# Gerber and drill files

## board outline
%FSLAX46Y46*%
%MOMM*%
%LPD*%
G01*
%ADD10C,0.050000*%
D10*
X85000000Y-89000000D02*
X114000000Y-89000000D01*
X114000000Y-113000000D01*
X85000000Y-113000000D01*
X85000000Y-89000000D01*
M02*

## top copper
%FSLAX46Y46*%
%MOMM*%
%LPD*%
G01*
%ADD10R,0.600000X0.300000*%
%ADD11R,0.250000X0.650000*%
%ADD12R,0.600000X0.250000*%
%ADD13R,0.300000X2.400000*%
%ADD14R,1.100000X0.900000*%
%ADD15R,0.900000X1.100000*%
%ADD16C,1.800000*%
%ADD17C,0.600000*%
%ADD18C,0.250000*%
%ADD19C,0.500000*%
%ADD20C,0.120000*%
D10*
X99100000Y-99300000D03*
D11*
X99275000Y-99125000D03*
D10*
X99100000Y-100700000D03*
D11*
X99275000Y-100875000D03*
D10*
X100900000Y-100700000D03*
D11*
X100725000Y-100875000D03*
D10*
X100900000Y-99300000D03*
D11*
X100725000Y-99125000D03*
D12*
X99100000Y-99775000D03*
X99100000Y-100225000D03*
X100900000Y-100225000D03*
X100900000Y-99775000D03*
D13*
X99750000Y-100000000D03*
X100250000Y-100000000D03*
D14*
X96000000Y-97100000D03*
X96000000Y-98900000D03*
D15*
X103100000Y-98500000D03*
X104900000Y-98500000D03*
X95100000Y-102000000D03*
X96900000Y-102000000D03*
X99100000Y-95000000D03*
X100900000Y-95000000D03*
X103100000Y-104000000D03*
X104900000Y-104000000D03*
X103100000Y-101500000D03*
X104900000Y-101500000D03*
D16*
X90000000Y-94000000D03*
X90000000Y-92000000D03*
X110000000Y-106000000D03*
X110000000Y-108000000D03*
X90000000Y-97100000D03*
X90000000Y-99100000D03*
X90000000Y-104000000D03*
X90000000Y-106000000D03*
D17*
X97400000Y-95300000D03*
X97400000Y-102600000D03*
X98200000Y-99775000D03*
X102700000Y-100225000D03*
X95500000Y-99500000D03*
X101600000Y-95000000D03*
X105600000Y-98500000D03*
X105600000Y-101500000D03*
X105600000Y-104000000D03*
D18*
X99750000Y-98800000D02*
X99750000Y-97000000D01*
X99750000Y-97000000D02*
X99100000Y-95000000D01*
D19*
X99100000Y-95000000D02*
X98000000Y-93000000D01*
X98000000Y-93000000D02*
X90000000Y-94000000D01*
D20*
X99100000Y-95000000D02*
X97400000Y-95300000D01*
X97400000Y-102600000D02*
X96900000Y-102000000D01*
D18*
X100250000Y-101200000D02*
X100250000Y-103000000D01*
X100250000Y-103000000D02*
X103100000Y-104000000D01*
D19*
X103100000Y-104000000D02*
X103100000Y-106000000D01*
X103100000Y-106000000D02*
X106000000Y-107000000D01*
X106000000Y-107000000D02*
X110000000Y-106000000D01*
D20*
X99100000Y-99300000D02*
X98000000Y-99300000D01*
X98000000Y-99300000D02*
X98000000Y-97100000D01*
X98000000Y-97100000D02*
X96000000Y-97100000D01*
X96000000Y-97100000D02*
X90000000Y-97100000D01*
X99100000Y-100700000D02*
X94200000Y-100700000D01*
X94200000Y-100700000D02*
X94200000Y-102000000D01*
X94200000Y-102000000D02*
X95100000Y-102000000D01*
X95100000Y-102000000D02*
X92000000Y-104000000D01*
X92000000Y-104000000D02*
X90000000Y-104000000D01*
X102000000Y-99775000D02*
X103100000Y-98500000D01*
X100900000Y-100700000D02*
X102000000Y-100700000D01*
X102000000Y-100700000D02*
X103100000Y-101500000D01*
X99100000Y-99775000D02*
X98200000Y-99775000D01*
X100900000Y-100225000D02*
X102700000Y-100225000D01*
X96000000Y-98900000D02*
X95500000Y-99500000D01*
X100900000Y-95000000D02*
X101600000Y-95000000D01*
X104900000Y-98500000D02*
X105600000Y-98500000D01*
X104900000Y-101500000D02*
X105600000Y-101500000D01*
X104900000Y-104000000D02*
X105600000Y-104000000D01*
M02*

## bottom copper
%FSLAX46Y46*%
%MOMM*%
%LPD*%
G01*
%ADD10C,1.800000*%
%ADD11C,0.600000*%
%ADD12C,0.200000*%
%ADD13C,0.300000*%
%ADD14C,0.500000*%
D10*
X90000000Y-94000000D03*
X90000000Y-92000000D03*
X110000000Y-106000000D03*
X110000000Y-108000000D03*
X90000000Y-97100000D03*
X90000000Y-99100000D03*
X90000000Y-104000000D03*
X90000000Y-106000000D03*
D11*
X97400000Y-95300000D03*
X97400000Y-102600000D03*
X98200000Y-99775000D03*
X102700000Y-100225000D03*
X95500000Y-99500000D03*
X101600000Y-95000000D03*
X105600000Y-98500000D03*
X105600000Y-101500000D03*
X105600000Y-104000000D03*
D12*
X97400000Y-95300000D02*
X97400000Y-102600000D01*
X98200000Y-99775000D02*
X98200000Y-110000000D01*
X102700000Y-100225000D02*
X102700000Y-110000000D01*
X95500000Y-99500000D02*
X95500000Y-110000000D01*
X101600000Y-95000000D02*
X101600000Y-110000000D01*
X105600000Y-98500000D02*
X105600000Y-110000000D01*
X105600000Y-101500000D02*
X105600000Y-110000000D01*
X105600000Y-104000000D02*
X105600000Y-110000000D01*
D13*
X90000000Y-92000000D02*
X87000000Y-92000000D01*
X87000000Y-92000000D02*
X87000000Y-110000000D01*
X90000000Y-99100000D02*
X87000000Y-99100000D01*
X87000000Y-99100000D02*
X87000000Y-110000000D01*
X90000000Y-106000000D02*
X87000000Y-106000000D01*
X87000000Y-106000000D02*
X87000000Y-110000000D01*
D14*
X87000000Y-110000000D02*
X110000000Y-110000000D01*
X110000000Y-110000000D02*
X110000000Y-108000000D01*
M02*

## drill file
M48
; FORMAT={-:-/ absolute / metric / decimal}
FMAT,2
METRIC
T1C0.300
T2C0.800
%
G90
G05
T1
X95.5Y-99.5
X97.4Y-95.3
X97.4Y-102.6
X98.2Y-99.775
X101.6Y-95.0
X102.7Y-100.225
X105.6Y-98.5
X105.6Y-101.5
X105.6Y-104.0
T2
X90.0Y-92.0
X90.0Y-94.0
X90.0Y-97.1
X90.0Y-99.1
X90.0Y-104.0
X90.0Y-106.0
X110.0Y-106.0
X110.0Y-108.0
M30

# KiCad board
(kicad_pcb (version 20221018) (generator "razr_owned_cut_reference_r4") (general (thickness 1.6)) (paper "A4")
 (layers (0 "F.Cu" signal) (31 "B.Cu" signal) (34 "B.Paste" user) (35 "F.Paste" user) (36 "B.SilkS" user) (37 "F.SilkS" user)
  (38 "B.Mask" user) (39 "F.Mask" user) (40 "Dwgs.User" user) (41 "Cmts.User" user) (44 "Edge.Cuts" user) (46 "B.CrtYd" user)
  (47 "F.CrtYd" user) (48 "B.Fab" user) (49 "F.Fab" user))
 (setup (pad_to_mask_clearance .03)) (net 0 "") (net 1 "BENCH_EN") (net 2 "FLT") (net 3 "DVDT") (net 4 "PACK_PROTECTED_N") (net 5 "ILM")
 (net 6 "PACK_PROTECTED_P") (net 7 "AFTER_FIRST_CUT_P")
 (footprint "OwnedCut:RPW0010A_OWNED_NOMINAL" (layer "F.Cu") (at 100 100)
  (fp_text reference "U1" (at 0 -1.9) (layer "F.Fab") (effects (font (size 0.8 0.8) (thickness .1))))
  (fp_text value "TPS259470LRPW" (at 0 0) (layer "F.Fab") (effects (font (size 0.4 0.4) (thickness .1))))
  (pad "1" smd rect (at -0.9 -0.7) (size 0.6 0.3) (layers "F.Cu" "F.Paste" "F.Mask") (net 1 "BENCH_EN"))
  (pad "1" smd rect (at -0.725 -0.875) (size 0.25 0.65) (layers "F.Cu" "F.Paste" "F.Mask") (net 1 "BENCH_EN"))
  (pad "4" smd rect (at -0.9 0.7) (size 0.6 0.3) (layers "F.Cu" "F.Paste" "F.Mask") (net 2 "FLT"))
  (pad "4" smd rect (at -0.725 0.875) (size 0.25 0.65) (layers "F.Cu" "F.Paste" "F.Mask") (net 2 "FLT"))
  (pad "7" smd rect (at 0.9 0.7) (size 0.6 0.3) (layers "F.Cu" "F.Paste" "F.Mask") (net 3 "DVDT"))
  (pad "7" smd rect (at 0.725 0.875) (size 0.25 0.65) (layers "F.Cu" "F.Paste" "F.Mask") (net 3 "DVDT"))
  (pad "10" smd rect (at 0.9 -0.7) (size 0.6 0.3) (layers "F.Cu" "F.Paste" "F.Mask"))
  (pad "10" smd rect (at 0.725 -0.875) (size 0.25 0.65) (layers "F.Cu" "F.Paste" "F.Mask"))
  (pad "2" smd rect (at -0.9 -0.225) (size 0.6 0.25) (layers "F.Cu" "F.Paste" "F.Mask") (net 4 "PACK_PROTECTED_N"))
  (pad "3" smd rect (at -0.9 0.225) (size 0.6 0.25) (layers "F.Cu" "F.Paste" "F.Mask"))
  (pad "8" smd rect (at 0.9 0.225) (size 0.6 0.25) (layers "F.Cu" "F.Paste" "F.Mask") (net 4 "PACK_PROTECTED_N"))
  (pad "9" smd rect (at 0.9 -0.225) (size 0.6 0.25) (layers "F.Cu" "F.Paste" "F.Mask") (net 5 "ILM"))
  (pad "5" smd rect (at -0.25 0) (size 0.3 2.4) (layers "F.Cu" "F.Paste" "F.Mask") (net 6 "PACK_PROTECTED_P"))
  (pad "6" smd rect (at 0.25 0) (size 0.3 2.4) (layers "F.Cu" "F.Paste" "F.Mask") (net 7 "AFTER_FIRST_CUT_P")))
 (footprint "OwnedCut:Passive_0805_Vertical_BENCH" (layer "F.Cu") (at 96 98)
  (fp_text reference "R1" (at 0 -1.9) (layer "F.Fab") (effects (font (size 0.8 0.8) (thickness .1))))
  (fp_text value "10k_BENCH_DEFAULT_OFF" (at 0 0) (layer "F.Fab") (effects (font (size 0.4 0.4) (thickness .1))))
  (pad "1" smd rect (at 0 -0.9) (size 1.1 0.9) (layers "F.Cu" "F.Paste" "F.Mask") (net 1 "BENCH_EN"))
  (pad "2" smd rect (at 0 0.9) (size 1.1 0.9) (layers "F.Cu" "F.Paste" "F.Mask") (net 4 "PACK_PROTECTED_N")))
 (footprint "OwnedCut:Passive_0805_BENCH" (layer "F.Cu") (at 104 98.5)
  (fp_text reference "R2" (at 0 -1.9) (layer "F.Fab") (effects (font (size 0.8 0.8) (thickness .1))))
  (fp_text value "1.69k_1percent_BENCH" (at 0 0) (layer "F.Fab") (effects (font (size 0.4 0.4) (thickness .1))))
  (pad "1" smd rect (at -0.9 0) (size 0.9 1.1) (layers "F.Cu" "F.Paste" "F.Mask") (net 5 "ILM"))
  (pad "2" smd rect (at 0.9 0) (size 0.9 1.1) (layers "F.Cu" "F.Paste" "F.Mask") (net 4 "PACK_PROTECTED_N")))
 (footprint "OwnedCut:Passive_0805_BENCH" (layer "F.Cu") (at 96 102)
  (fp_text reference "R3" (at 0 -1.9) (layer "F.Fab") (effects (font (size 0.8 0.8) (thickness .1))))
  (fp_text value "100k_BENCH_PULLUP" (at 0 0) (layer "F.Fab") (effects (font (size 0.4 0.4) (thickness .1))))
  (pad "1" smd rect (at -0.9 0) (size 0.9 1.1) (layers "F.Cu" "F.Paste" "F.Mask") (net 2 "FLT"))
  (pad "2" smd rect (at 0.9 0) (size 0.9 1.1) (layers "F.Cu" "F.Paste" "F.Mask") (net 6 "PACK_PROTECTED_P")))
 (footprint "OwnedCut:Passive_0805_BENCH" (layer "F.Cu") (at 100 95)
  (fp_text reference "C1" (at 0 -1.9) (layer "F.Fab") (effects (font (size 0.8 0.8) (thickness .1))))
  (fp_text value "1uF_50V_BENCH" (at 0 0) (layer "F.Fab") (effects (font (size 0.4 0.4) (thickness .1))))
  (pad "1" smd rect (at -0.9 0) (size 0.9 1.1) (layers "F.Cu" "F.Paste" "F.Mask") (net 6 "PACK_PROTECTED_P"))
  (pad "2" smd rect (at 0.9 0) (size 0.9 1.1) (layers "F.Cu" "F.Paste" "F.Mask") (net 4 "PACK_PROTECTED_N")))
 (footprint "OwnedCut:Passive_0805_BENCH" (layer "F.Cu") (at 104 104)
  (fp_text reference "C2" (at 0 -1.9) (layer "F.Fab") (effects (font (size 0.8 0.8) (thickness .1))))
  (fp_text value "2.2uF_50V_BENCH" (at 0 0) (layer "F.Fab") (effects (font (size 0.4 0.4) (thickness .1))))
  (pad "1" smd rect (at -0.9 0) (size 0.9 1.1) (layers "F.Cu" "F.Paste" "F.Mask") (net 7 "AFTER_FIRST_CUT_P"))
  (pad "2" smd rect (at 0.9 0) (size 0.9 1.1) (layers "F.Cu" "F.Paste" "F.Mask") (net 4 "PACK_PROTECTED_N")))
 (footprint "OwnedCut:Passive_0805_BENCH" (layer "F.Cu") (at 104 101.5)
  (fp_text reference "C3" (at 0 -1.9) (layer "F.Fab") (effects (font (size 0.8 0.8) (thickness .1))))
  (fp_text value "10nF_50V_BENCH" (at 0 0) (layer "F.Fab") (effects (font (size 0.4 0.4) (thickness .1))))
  (pad "1" smd rect (at -0.9 0) (size 0.9 1.1) (layers "F.Cu" "F.Paste" "F.Mask") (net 3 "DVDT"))
  (pad "2" smd rect (at 0.9 0) (size 0.9 1.1) (layers "F.Cu" "F.Paste" "F.Mask") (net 4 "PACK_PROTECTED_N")))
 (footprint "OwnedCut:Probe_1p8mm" (layer "F.Cu") (at 90 94)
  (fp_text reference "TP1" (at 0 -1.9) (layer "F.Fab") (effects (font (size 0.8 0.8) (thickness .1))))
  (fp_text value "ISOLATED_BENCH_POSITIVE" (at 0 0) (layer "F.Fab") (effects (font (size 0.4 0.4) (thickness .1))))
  (pad "1" thru_hole circle (at 0 0) (size 1.8 1.8) (drill .8) (layers "*.Cu" "*.Mask") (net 6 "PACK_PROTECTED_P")))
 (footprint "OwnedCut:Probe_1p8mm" (layer "F.Cu") (at 90 92)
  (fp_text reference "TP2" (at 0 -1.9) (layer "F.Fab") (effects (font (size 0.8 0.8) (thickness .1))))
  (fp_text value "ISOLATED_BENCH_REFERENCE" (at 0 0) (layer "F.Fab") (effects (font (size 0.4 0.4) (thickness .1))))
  (pad "1" thru_hole circle (at 0 0) (size 1.8 1.8) (drill .8) (layers "*.Cu" "*.Mask") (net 4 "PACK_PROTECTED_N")))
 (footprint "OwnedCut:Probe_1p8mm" (layer "F.Cu") (at 110 106)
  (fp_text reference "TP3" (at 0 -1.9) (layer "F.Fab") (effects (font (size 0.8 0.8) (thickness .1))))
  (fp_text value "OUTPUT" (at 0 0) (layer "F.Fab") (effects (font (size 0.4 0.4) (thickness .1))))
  (pad "1" thru_hole circle (at 0 0) (size 1.8 1.8) (drill .8) (layers "*.Cu" "*.Mask") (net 7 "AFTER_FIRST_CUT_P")))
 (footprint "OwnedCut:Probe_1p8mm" (layer "F.Cu") (at 110 108)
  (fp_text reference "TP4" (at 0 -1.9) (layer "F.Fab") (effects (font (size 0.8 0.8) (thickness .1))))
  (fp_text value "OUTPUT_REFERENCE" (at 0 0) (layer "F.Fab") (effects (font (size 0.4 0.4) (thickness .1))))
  (pad "1" thru_hole circle (at 0 0) (size 1.8 1.8) (drill .8) (layers "*.Cu" "*.Mask") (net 4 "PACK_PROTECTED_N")))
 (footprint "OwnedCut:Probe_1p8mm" (layer "F.Cu") (at 90 97.1)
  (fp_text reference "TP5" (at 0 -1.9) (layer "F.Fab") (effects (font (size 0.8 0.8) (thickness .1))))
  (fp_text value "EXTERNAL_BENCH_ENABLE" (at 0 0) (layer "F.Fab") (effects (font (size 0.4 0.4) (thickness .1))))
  (pad "1" thru_hole circle (at 0 0) (size 1.8 1.8) (drill .8) (layers "*.Cu" "*.Mask") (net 1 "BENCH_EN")))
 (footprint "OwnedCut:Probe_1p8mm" (layer "F.Cu") (at 90 99.1)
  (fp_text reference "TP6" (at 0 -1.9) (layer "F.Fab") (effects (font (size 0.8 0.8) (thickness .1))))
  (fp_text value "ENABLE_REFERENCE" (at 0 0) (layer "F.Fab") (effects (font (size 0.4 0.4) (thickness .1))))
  (pad "1" thru_hole circle (at 0 0) (size 1.8 1.8) (drill .8) (layers "*.Cu" "*.Mask") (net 4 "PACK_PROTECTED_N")))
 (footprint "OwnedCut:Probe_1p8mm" (layer "F.Cu") (at 90 104)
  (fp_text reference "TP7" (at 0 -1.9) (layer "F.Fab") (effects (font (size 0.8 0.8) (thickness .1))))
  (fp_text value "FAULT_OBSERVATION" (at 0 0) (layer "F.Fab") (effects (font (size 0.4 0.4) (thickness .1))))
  (pad "1" thru_hole circle (at 0 0) (size 1.8 1.8) (drill .8) (layers "*.Cu" "*.Mask") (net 2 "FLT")))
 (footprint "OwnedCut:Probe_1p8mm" (layer "F.Cu") (at 90 106)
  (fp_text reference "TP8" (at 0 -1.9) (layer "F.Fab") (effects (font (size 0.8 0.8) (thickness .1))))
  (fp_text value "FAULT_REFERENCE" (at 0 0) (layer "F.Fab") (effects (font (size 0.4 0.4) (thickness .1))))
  (pad "1" thru_hole circle (at 0 0) (size 1.8 1.8) (drill .8) (layers "*.Cu" "*.Mask") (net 4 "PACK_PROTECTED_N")))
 (segment (start 99.75 98.8) (end 99.75 97) (width 0.25) (layer "F.Cu") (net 6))
 (segment (start 99.75 97) (end 99.1 95) (width 0.25) (layer "F.Cu") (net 6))
 (segment (start 99.1 95) (end 98 93) (width 0.5) (layer "F.Cu") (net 6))
 (segment (start 98 93) (end 90 94) (width 0.5) (layer "F.Cu") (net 6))
 (segment (start 99.1 95) (end 97.4 95.3) (width 0.12) (layer "F.Cu") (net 6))
 (via (at 97.4 95.3) (size .6) (drill .3) (layers "F.Cu" "B.Cu") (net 6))
 (segment (start 97.4 95.3) (end 97.4 102.6) (width 0.2) (layer "B.Cu") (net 6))
 (via (at 97.4 102.6) (size .6) (drill .3) (layers "F.Cu" "B.Cu") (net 6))
 (segment (start 97.4 102.6) (end 96.9 102) (width 0.12) (layer "F.Cu") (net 6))
 (segment (start 100.25 101.2) (end 100.25 103) (width 0.25) (layer "F.Cu") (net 7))
 (segment (start 100.25 103) (end 103.1 104) (width 0.25) (layer "F.Cu") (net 7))
 (segment (start 103.1 104) (end 103.1 106) (width 0.5) (layer "F.Cu") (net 7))
 (segment (start 103.1 106) (end 106 107) (width 0.5) (layer "F.Cu") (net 7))
 (segment (start 106 107) (end 110 106) (width 0.5) (layer "F.Cu") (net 7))
 (segment (start 99.1 99.3) (end 98 99.3) (width 0.12) (layer "F.Cu") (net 1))
 (segment (start 98 99.3) (end 98 97.1) (width 0.12) (layer "F.Cu") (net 1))
 (segment (start 98 97.1) (end 96 97.1) (width 0.12) (layer "F.Cu") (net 1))
 (segment (start 96 97.1) (end 90 97.1) (width 0.12) (layer "F.Cu") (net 1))
 (segment (start 99.1 100.7) (end 94.2 100.7) (width 0.12) (layer "F.Cu") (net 2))
 (segment (start 94.2 100.7) (end 94.2 102) (width 0.12) (layer "F.Cu") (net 2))
 (segment (start 94.2 102) (end 95.1 102) (width 0.12) (layer "F.Cu") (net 2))
 (segment (start 95.1 102) (end 92 104) (width 0.12) (layer "F.Cu") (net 2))
 (segment (start 92 104) (end 90 104) (width 0.12) (layer "F.Cu") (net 2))
 (segment (start 102 99.775) (end 103.1 98.5) (width 0.12) (layer "F.Cu") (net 5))
 (segment (start 100.9 100.7) (end 102 100.7) (width 0.12) (layer "F.Cu") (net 3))
 (segment (start 102 100.7) (end 103.1 101.5) (width 0.12) (layer "F.Cu") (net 3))
 (segment (start 99.1 99.775) (end 98.2 99.775) (width 0.12) (layer "F.Cu") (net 4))
 (via (at 98.2 99.775) (size .6) (drill .3) (layers "F.Cu" "B.Cu") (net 4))
 (segment (start 98.2 99.775) (end 98.2 110) (width 0.2) (layer "B.Cu") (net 4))
 (segment (start 100.9 100.225) (end 102.7 100.225) (width 0.12) (layer "F.Cu") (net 4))
 (via (at 102.7 100.225) (size .6) (drill .3) (layers "F.Cu" "B.Cu") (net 4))
 (segment (start 102.7 100.225) (end 102.7 110) (width 0.2) (layer "B.Cu") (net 4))
 (segment (start 96 98.9) (end 95.5 99.5) (width 0.12) (layer "F.Cu") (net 4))
 (via (at 95.5 99.5) (size .6) (drill .3) (layers "F.Cu" "B.Cu") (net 4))
 (segment (start 95.5 99.5) (end 95.5 110) (width 0.2) (layer "B.Cu") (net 4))
 (segment (start 100.9 95) (end 101.6 95) (width 0.12) (layer "F.Cu") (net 4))
 (via (at 101.6 95) (size .6) (drill .3) (layers "F.Cu" "B.Cu") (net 4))
 (segment (start 101.6 95) (end 101.6 110) (width 0.2) (layer "B.Cu") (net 4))
 (segment (start 104.9 98.5) (end 105.6 98.5) (width 0.12) (layer "F.Cu") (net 4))
 (via (at 105.6 98.5) (size .6) (drill .3) (layers "F.Cu" "B.Cu") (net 4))
 (segment (start 105.6 98.5) (end 105.6 110) (width 0.2) (layer "B.Cu") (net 4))
 (segment (start 104.9 101.5) (end 105.6 101.5) (width 0.12) (layer "F.Cu") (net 4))
 (via (at 105.6 101.5) (size .6) (drill .3) (layers "F.Cu" "B.Cu") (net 4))
 (segment (start 105.6 101.5) (end 105.6 110) (width 0.2) (layer "B.Cu") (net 4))
 (segment (start 104.9 104) (end 105.6 104) (width 0.12) (layer "F.Cu") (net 4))
 (via (at 105.6 104) (size .6) (drill .3) (layers "F.Cu" "B.Cu") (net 4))
 (segment (start 105.6 104) (end 105.6 110) (width 0.2) (layer "B.Cu") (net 4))
 (segment (start 90 92) (end 87 92) (width 0.3) (layer "B.Cu") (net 4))
 (segment (start 87 92) (end 87 110) (width 0.3) (layer "B.Cu") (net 4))
 (segment (start 90 99.1) (end 87 99.1) (width 0.3) (layer "B.Cu") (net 4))
 (segment (start 87 99.1) (end 87 110) (width 0.3) (layer "B.Cu") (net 4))
 (segment (start 90 106) (end 87 106) (width 0.3) (layer "B.Cu") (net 4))
 (segment (start 87 106) (end 87 110) (width 0.3) (layer "B.Cu") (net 4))
 (segment (start 87 110) (end 110 110) (width 0.5) (layer "B.Cu") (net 4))
 (segment (start 110 110) (end 110 108) (width 0.5) (layer "B.Cu") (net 4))
 (gr_rect (start 85 89) (end 114 113) (stroke (width .05) (type default)) (fill none) (layer "Edge.Cuts")))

